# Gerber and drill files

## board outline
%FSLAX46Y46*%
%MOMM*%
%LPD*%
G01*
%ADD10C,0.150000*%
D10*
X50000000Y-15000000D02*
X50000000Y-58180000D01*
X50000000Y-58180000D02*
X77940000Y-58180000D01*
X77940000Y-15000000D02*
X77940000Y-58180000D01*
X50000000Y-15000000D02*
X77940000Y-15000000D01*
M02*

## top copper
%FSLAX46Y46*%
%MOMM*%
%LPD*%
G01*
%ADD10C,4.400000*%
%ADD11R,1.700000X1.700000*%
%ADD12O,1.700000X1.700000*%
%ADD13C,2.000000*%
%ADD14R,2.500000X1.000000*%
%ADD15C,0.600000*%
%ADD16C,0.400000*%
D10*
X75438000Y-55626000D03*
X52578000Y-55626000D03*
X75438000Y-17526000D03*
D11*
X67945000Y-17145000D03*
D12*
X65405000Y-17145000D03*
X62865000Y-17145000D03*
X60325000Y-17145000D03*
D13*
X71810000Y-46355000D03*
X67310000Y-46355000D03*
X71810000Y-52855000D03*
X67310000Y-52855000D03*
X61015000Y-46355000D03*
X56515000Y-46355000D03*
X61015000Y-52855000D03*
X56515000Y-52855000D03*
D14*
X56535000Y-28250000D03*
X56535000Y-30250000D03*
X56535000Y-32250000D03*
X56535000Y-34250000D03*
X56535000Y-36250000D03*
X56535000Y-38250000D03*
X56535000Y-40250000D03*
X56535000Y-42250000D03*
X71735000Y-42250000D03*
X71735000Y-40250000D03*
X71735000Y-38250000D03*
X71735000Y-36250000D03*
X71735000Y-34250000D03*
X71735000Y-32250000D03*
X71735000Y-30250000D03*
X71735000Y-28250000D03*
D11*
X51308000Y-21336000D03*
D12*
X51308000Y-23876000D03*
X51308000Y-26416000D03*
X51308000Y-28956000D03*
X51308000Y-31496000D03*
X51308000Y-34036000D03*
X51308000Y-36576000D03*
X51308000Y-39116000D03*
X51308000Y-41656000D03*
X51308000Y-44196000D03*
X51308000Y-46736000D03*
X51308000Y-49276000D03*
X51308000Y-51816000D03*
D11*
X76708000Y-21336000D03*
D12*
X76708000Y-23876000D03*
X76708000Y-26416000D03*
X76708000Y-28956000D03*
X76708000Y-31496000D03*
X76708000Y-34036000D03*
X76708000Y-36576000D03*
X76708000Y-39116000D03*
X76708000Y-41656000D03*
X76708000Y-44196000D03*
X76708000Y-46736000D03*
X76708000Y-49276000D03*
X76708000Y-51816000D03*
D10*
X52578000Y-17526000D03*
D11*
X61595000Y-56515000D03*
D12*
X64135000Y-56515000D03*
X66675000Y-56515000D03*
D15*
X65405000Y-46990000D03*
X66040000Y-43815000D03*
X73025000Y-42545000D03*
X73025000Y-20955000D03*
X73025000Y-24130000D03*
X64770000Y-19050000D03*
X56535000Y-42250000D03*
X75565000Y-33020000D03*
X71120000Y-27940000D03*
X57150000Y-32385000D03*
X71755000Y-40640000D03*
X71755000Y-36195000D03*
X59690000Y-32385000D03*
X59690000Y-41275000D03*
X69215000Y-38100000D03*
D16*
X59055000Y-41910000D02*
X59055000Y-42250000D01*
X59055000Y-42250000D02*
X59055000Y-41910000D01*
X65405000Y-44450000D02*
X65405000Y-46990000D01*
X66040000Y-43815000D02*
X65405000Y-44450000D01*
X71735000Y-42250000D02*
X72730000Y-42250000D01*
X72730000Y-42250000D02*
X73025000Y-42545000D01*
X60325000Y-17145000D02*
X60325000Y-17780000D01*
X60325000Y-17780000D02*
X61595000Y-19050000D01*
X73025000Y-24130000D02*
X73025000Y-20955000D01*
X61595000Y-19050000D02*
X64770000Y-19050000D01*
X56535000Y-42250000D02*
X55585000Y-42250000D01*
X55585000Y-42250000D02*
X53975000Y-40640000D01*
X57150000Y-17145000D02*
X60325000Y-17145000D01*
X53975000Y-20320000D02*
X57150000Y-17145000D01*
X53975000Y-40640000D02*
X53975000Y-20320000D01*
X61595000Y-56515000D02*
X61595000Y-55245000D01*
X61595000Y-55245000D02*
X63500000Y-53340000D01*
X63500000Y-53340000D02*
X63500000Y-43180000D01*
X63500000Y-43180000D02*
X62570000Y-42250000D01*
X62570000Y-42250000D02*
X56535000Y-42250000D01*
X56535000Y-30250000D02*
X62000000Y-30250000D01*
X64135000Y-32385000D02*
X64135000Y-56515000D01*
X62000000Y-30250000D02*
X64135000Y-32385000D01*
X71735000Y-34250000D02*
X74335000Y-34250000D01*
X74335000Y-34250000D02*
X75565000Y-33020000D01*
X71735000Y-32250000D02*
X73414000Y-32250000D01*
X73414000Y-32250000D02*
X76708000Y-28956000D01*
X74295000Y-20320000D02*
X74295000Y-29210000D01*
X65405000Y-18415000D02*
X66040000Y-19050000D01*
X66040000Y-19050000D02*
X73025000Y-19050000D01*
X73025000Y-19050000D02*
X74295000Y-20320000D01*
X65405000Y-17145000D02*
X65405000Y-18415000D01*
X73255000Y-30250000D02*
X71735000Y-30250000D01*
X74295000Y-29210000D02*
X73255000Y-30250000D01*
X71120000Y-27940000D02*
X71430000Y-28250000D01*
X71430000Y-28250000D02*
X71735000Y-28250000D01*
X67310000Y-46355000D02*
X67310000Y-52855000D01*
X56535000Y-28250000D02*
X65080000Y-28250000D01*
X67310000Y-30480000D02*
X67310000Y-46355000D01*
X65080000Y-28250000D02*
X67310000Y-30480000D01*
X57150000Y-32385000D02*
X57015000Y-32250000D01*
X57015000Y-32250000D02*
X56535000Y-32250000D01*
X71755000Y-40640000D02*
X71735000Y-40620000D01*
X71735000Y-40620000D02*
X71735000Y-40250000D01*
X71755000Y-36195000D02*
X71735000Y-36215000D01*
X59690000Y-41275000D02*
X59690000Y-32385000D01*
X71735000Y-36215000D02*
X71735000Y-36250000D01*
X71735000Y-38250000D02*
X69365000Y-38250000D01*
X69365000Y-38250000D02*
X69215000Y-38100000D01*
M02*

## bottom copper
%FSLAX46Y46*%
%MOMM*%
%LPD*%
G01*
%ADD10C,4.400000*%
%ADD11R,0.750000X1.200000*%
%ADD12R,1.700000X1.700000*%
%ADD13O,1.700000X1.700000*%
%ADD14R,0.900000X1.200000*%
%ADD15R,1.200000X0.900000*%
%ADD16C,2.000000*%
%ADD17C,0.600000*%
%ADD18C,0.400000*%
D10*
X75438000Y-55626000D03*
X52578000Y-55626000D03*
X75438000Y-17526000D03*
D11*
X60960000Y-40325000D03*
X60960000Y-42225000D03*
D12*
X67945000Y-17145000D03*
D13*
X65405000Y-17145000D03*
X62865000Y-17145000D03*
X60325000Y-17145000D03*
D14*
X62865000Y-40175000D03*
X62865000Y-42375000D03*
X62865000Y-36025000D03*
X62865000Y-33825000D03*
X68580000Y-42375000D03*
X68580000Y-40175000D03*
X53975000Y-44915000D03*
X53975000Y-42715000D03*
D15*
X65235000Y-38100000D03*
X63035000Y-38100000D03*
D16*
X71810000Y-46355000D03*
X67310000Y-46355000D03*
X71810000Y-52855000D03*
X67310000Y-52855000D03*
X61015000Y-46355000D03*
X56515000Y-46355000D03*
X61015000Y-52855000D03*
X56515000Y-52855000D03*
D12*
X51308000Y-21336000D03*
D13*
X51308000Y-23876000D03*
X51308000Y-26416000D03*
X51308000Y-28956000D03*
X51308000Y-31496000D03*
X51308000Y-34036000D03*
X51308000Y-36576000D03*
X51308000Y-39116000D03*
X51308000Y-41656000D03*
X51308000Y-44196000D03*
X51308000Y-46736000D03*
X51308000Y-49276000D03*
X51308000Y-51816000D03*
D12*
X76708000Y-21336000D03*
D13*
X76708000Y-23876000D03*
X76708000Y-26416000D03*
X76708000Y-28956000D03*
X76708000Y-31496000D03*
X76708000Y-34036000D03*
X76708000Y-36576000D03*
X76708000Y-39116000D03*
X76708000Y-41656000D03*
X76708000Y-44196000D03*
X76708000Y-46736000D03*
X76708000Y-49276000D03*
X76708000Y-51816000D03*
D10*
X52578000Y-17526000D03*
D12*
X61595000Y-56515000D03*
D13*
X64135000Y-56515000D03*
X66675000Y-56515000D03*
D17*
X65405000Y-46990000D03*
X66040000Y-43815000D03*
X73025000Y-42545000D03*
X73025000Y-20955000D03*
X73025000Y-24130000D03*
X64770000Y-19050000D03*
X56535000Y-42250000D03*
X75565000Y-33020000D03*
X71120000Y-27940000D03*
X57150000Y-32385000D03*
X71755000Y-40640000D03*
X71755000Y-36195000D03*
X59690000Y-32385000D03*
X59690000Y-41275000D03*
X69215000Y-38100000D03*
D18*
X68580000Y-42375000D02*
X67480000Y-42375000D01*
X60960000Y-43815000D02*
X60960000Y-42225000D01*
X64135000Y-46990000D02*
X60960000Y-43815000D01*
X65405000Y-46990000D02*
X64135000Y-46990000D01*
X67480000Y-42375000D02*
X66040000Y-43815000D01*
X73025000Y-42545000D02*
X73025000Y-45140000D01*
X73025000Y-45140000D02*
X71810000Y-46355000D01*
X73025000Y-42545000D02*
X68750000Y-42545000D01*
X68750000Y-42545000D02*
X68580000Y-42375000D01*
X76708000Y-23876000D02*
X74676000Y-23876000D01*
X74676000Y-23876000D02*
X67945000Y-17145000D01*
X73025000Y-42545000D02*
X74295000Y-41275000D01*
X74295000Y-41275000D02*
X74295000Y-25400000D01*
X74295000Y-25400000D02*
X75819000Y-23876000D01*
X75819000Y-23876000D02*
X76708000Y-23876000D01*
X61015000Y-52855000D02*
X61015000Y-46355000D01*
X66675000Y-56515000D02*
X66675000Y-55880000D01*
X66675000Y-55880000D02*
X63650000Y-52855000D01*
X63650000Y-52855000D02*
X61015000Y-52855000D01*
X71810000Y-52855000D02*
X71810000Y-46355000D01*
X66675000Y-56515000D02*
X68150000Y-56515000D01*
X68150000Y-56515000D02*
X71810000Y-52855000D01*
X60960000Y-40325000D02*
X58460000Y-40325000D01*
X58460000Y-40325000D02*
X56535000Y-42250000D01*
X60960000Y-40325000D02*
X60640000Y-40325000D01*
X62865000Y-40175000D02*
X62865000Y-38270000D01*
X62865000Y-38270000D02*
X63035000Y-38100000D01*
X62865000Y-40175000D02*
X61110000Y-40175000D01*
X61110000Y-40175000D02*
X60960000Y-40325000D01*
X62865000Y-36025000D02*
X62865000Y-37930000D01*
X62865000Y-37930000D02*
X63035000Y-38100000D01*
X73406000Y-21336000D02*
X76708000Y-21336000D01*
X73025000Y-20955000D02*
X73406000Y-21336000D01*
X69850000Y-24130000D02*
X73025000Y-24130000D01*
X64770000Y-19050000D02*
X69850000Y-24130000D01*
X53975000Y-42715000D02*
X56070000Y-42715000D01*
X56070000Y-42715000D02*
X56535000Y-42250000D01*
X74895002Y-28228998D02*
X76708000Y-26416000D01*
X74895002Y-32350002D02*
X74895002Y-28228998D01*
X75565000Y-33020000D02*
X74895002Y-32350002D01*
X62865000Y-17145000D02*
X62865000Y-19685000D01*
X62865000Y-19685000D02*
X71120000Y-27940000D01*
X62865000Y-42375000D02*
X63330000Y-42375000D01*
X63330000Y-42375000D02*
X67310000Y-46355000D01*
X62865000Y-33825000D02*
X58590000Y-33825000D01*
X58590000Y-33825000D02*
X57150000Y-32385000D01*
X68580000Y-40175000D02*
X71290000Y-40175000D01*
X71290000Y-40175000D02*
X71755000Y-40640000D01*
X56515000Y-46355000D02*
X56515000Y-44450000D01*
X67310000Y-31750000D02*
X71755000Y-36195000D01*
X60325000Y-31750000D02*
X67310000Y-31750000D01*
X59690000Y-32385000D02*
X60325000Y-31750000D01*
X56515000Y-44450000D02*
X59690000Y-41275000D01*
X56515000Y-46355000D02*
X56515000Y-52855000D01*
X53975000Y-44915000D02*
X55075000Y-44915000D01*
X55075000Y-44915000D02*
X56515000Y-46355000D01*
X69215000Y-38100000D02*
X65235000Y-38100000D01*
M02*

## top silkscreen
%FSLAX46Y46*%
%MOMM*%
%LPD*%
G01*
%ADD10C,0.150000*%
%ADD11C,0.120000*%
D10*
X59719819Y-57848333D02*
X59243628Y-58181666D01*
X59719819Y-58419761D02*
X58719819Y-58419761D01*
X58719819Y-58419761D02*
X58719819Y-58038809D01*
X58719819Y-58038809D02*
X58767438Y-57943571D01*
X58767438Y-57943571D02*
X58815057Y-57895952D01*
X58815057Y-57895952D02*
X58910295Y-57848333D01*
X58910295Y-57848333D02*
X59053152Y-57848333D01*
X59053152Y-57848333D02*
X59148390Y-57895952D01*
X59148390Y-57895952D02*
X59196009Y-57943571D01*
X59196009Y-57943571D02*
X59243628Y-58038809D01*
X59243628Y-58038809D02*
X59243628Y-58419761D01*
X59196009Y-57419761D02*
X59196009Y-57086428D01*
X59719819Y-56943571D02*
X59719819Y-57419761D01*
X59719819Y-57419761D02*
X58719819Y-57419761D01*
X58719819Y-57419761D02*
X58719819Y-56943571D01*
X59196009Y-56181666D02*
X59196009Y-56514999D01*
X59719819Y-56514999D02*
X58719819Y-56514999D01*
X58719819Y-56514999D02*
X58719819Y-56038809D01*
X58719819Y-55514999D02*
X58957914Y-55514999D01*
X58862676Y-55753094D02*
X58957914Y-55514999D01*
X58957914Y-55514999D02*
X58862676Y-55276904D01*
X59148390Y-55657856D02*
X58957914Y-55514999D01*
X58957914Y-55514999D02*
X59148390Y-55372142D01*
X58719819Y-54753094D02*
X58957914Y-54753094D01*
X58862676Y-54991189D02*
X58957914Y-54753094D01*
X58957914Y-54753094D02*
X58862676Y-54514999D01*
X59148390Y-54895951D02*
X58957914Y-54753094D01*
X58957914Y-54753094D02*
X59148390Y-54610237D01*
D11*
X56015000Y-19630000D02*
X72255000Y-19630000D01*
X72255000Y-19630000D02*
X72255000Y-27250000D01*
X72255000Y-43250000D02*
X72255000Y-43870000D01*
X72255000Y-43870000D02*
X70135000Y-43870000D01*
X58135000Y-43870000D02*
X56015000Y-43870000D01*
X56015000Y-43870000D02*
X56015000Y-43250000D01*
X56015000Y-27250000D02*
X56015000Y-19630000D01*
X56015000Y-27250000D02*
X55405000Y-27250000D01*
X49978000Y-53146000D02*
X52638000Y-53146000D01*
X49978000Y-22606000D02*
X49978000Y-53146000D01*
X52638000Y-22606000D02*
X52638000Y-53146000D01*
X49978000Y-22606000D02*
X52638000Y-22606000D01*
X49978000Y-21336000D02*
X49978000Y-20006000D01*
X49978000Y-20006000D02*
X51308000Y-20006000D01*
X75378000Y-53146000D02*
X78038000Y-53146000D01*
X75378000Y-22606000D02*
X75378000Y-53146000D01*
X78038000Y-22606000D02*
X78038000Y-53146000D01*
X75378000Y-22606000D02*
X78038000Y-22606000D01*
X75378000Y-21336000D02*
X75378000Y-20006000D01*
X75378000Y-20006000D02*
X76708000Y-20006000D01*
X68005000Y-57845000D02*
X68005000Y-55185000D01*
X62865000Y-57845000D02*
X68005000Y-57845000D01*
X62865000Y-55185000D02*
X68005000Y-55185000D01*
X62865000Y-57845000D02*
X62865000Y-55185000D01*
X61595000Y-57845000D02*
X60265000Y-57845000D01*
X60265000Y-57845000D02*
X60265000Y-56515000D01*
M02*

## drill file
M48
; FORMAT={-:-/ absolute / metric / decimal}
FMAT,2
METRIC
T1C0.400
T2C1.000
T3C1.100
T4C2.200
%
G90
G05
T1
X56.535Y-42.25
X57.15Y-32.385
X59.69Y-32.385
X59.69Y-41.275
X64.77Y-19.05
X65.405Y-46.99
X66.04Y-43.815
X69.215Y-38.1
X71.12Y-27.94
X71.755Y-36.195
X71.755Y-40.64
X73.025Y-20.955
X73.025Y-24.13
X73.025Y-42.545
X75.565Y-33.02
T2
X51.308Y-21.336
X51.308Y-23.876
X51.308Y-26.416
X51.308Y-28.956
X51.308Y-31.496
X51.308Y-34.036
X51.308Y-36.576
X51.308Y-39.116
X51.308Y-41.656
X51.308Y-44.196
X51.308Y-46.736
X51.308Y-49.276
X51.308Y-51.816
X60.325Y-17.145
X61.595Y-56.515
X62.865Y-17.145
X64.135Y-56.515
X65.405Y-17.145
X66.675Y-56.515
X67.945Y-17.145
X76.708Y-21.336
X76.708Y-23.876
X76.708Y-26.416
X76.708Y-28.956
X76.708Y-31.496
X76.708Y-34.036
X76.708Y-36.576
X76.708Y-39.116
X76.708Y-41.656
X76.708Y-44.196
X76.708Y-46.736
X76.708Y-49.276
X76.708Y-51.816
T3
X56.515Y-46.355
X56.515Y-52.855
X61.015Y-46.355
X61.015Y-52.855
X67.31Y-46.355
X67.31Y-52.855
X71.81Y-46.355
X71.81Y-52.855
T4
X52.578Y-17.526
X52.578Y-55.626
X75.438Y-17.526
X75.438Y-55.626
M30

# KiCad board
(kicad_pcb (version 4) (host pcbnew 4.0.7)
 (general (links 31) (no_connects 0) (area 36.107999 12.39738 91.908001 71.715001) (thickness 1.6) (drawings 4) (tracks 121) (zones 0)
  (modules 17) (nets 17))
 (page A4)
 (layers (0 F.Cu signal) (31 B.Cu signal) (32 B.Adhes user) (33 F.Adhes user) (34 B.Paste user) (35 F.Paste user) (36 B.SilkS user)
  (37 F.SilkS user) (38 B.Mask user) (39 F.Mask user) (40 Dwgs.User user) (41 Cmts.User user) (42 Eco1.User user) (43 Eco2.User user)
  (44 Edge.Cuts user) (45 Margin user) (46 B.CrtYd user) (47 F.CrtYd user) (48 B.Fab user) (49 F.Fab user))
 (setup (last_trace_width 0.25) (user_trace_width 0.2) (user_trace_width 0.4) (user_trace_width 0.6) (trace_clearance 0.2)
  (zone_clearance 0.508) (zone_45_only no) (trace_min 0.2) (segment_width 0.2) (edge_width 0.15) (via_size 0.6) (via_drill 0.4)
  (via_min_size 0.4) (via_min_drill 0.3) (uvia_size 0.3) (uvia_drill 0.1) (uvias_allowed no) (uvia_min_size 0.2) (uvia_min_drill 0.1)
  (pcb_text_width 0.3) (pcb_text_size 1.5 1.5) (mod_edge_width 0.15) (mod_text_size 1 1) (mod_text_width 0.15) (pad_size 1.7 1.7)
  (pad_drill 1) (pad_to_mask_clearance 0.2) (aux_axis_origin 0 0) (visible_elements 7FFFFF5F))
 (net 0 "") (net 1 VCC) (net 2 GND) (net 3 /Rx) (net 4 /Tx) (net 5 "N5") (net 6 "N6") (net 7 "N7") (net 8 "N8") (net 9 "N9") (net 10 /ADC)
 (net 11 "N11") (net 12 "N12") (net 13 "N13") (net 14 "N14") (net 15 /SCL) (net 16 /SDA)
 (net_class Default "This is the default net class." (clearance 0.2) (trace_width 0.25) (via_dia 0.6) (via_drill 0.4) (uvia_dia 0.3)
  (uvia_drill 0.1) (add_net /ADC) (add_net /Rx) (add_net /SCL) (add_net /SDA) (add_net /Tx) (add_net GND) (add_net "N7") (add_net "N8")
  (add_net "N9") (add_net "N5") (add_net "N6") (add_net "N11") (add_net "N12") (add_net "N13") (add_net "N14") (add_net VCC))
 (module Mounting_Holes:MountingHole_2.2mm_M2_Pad (layer F.Cu) (at 75.438 55.626)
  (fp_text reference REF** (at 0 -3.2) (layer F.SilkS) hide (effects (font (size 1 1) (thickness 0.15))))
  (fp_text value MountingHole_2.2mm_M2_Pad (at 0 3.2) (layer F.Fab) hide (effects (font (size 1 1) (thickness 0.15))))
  (pad 1 thru_hole circle (at 0 0) (size 4.4 4.4) (drill 2.2) (layers *.Cu *.Mask)))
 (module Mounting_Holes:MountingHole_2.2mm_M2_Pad (layer F.Cu) (at 52.578 55.626)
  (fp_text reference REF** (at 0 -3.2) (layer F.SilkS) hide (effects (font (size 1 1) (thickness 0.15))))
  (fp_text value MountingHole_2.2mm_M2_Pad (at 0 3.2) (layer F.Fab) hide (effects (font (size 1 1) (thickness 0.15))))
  (pad 1 thru_hole circle (at 0 0) (size 4.4 4.4) (drill 2.2) (layers *.Cu *.Mask)))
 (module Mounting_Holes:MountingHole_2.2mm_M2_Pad (layer F.Cu) (at 75.438 17.526)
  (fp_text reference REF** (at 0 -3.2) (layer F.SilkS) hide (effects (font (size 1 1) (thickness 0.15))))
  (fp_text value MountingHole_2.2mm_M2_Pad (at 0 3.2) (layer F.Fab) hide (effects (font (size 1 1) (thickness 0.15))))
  (pad 1 thru_hole circle (at 0 0) (size 4.4 4.4) (drill 2.2) (layers *.Cu *.Mask)))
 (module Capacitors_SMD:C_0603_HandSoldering (layer B.Cu) (at 60.96 41.275 270)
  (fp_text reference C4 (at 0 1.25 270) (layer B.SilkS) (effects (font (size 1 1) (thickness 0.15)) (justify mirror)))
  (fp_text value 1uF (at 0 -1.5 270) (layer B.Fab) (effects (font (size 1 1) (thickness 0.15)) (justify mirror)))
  (pad 1 smd rect (at -0.95 0 270) (size 1.2 0.75) (layers B.Cu B.Paste B.Mask) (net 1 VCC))
  (pad 2 smd rect (at 0.95 0 270) (size 1.2 0.75) (layers B.Cu B.Paste B.Mask) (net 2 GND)))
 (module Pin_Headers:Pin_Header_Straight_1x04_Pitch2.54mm (layer B.Cu) (at 67.945 17.145 90)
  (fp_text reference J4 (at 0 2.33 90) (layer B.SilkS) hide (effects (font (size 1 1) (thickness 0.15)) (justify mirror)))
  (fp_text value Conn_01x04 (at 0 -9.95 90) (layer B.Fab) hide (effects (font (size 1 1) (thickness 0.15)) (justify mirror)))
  (pad 1 thru_hole rect (at 0 0 90) (size 1.7 1.7) (drill 1) (layers *.Cu *.Mask) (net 2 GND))
  (pad 2 thru_hole oval (at 0 -2.54 90) (size 1.7 1.7) (drill 1) (layers *.Cu *.Mask) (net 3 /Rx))
  (pad 3 thru_hole oval (at 0 -5.08 90) (size 1.7 1.7) (drill 1) (layers *.Cu *.Mask) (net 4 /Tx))
  (pad 4 thru_hole oval (at 0 -7.62 90) (size 1.7 1.7) (drill 1) (layers *.Cu *.Mask) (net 1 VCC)))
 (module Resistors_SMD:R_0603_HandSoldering (layer B.Cu) (at 62.865 41.275 270)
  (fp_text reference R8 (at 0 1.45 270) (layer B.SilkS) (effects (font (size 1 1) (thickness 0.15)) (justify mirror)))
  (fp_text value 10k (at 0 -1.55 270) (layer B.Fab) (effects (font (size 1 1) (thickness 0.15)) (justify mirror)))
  (pad 1 smd rect (at -1.1 0 270) (size 1.2 0.9) (layers B.Cu B.Paste B.Mask) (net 1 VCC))
  (pad 2 smd rect (at 1.1 0 270) (size 1.2 0.9) (layers B.Cu B.Paste B.Mask) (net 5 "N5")))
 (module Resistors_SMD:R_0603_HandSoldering (layer B.Cu) (at 62.865 34.925 90)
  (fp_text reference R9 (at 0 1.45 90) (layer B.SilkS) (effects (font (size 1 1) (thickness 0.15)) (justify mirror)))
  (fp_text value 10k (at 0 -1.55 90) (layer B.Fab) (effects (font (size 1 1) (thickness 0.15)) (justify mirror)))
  (pad 1 smd rect (at -1.1 0 90) (size 1.2 0.9) (layers B.Cu B.Paste B.Mask) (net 1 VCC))
  (pad 2 smd rect (at 1.1 0 90) (size 1.2 0.9) (layers B.Cu B.Paste B.Mask) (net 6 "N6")))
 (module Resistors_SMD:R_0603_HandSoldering (layer B.Cu) (at 68.58 41.275 90)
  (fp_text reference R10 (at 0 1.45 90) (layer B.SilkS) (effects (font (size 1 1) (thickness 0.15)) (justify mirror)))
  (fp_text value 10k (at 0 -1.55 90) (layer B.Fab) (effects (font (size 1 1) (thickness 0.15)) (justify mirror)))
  (pad 1 smd rect (at -1.1 0 90) (size 1.2 0.9) (layers B.Cu B.Paste B.Mask) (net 2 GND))
  (pad 2 smd rect (at 1.1 0 90) (size 1.2 0.9) (layers B.Cu B.Paste B.Mask) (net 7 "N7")))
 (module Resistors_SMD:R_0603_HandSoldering (layer B.Cu) (at 53.975 43.815 90)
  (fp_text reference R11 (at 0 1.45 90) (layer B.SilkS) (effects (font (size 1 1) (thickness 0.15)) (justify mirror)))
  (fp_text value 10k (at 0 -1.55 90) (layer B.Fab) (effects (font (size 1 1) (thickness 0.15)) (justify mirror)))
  (pad 1 smd rect (at -1.1 0 90) (size 1.2 0.9) (layers B.Cu B.Paste B.Mask) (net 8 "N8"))
  (pad 2 smd rect (at 1.1 0 90) (size 1.2 0.9) (layers B.Cu B.Paste B.Mask) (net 1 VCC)))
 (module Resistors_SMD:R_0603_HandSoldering (layer B.Cu) (at 64.135 38.1 180)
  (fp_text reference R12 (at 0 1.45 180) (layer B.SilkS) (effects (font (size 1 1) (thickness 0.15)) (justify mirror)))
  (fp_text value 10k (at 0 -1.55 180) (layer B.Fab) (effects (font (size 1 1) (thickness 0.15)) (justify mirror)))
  (pad 1 smd rect (at -1.1 0 180) (size 1.2 0.9) (layers B.Cu B.Paste B.Mask) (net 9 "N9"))
  (pad 2 smd rect (at 1.1 0 180) (size 1.2 0.9) (layers B.Cu B.Paste B.Mask) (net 1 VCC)))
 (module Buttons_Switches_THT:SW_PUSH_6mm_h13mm (layer B.Cu) (at 67.31 46.355 270)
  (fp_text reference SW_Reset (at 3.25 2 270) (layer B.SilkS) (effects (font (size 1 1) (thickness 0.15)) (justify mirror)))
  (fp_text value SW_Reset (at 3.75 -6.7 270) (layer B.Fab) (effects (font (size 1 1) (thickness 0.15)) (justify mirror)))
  (pad 2 thru_hole circle (at 0 -4.5 180) (size 2 2) (drill 1.1) (layers *.Cu *.Mask) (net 2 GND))
  (pad 1 thru_hole circle (at 0 0 180) (size 2 2) (drill 1.1) (layers *.Cu *.Mask) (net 5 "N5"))
  (pad 2 thru_hole circle (at 6.5 -4.5 180) (size 2 2) (drill 1.1) (layers *.Cu *.Mask) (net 2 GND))
  (pad 1 thru_hole circle (at 6.5 0 180) (size 2 2) (drill 1.1) (layers *.Cu *.Mask) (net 5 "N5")))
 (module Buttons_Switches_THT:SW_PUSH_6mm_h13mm (layer B.Cu) (at 56.515 46.355 270)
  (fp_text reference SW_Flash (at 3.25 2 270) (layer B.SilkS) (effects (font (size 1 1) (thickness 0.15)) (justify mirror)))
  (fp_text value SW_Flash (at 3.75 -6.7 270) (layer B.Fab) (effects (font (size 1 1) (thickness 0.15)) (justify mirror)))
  (pad 2 thru_hole circle (at 0 -4.5 180) (size 2 2) (drill 1.1) (layers *.Cu *.Mask) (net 2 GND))
  (pad 1 thru_hole circle (at 0 0 180) (size 2 2) (drill 1.1) (layers *.Cu *.Mask) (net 8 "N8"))
  (pad 2 thru_hole circle (at 6.5 -4.5 180) (size 2 2) (drill 1.1) (layers *.Cu *.Mask) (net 2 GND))
  (pad 1 thru_hole circle (at 6.5 0 180) (size 2 2) (drill 1.1) (layers *.Cu *.Mask) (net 8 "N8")))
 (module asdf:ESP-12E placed (layer F.Cu) (at 64.135 31.75)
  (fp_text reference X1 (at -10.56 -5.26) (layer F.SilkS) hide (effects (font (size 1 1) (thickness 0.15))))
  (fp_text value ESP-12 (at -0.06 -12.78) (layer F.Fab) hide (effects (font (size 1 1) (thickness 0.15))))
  (fp_line (start -8.12 -12.12) (end 8.12 -12.12) (layer F.SilkS) (width 0.12))
  (fp_line (start 8.12 -12.12) (end 8.12 -4.5) (layer F.SilkS) (width 0.12))
  (fp_line (start 8.12 11.5) (end 8.12 12.12) (layer F.SilkS) (width 0.12))
  (fp_line (start 8.12 12.12) (end 6 12.12) (layer F.SilkS) (width 0.12))
  (fp_line (start -6 12.12) (end -8.12 12.12) (layer F.SilkS) (width 0.12))
  (fp_line (start -8.12 12.12) (end -8.12 11.5) (layer F.SilkS) (width 0.12))
  (fp_line (start -8.12 -4.5) (end -8.12 -12.12) (layer F.SilkS) (width 0.12))
  (fp_line (start -8.12 -4.5) (end -8.73 -4.5) (layer F.SilkS) (width 0.12))
  (pad 1 smd rect (at -7.6 -3.5) (size 2.5 1) (layers F.Cu F.Paste F.Mask) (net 5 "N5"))
  (pad 2 smd rect (at -7.6 -1.5) (size 2.5 1) (layers F.Cu F.Paste F.Mask) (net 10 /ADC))
  (pad 3 smd rect (at -7.6 0.5) (size 2.5 1) (layers F.Cu F.Paste F.Mask) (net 6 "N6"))
  (pad 4 smd rect (at -7.6 2.5) (size 2.5 1) (layers F.Cu F.Paste F.Mask) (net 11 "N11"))
  (pad 5 smd rect (at -7.6 4.5) (size 2.5 1) (layers F.Cu F.Paste F.Mask) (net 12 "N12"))
  (pad 6 smd rect (at -7.6 6.5) (size 2.5 1) (layers F.Cu F.Paste F.Mask) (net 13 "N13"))
  (pad 7 smd rect (at -7.6 8.5) (size 2.5 1) (layers F.Cu F.Paste F.Mask) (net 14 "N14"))
  (pad 8 smd rect (at -7.6 10.5) (size 2.5 1) (layers F.Cu F.Paste F.Mask) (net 1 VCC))
  (pad 9 smd rect (at 7.6 10.5) (size 2.5 1) (layers F.Cu F.Paste F.Mask) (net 2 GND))
  (pad 10 smd rect (at 7.6 8.5) (size 2.5 1) (layers F.Cu F.Paste F.Mask) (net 7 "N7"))
  (pad 11 smd rect (at 7.6 6.5) (size 2.5 1) (layers F.Cu F.Paste F.Mask) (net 9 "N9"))
  (pad 12 smd rect (at 7.6 4.5) (size 2.5 1) (layers F.Cu F.Paste F.Mask) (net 8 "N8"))
  (pad 13 smd rect (at 7.6 2.5) (size 2.5 1) (layers F.Cu F.Paste F.Mask) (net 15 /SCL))
  (pad 14 smd rect (at 7.6 0.5) (size 2.5 1) (layers F.Cu F.Paste F.Mask) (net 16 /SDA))
  (pad 15 smd rect (at 7.6 -1.5) (size 2.5 1) (layers F.Cu F.Paste F.Mask) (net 3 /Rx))
  (pad 16 smd rect (at 7.6 -3.5) (size 2.5 1) (layers F.Cu F.Paste F.Mask) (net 4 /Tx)))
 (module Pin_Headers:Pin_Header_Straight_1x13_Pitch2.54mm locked (layer F.Cu) (at 51.308 21.336)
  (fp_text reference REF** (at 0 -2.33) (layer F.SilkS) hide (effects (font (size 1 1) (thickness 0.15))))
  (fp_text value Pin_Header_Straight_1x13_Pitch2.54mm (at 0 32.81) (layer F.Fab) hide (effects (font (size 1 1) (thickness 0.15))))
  (fp_line (start -1.33 31.81) (end 1.33 31.81) (layer F.SilkS) (width 0.12))
  (fp_line (start -1.33 1.27) (end -1.33 31.81) (layer F.SilkS) (width 0.12))
  (fp_line (start 1.33 1.27) (end 1.33 31.81) (layer F.SilkS) (width 0.12))
  (fp_line (start -1.33 1.27) (end 1.33 1.27) (layer F.SilkS) (width 0.12))
  (fp_line (start -1.33 0) (end -1.33 -1.33) (layer F.SilkS) (width 0.12))
  (fp_line (start -1.33 -1.33) (end 0 -1.33) (layer F.SilkS) (width 0.12))
  (pad 1 thru_hole rect (at 0 0) (size 1.7 1.7) (drill 1) (layers *.Cu *.Mask))
  (pad 2 thru_hole oval (at 0 2.54) (size 1.7 1.7) (drill 1) (layers *.Cu *.Mask))
  (pad 3 thru_hole oval (at 0 5.08) (size 1.7 1.7) (drill 1) (layers *.Cu *.Mask))
  (pad 4 thru_hole oval (at 0 7.62) (size 1.7 1.7) (drill 1) (layers *.Cu *.Mask))
  (pad 5 thru_hole oval (at 0 10.16) (size 1.7 1.7) (drill 1) (layers *.Cu *.Mask))
  (pad 6 thru_hole oval (at 0 12.7) (size 1.7 1.7) (drill 1) (layers *.Cu *.Mask))
  (pad 7 thru_hole oval (at 0 15.24) (size 1.7 1.7) (drill 1) (layers *.Cu *.Mask))
  (pad 8 thru_hole oval (at 0 17.78) (size 1.7 1.7) (drill 1) (layers *.Cu *.Mask))
  (pad 9 thru_hole oval (at 0 20.32) (size 1.7 1.7) (drill 1) (layers *.Cu *.Mask))
  (pad 10 thru_hole oval (at 0 22.86) (size 1.7 1.7) (drill 1) (layers *.Cu *.Mask))
  (pad 11 thru_hole oval (at 0 25.4) (size 1.7 1.7) (drill 1) (layers *.Cu *.Mask))
  (pad 12 thru_hole oval (at 0 27.94) (size 1.7 1.7) (drill 1) (layers *.Cu *.Mask))
  (pad 13 thru_hole oval (at 0 30.48) (size 1.7 1.7) (drill 1) (layers *.Cu *.Mask)))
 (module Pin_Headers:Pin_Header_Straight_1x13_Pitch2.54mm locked (layer F.Cu) (at 76.708 21.336)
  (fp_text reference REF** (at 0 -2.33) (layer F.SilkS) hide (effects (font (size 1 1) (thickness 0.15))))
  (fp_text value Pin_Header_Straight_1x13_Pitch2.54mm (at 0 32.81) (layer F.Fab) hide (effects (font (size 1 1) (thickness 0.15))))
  (fp_line (start -1.33 31.81) (end 1.33 31.81) (layer F.SilkS) (width 0.12))
  (fp_line (start -1.33 1.27) (end -1.33 31.81) (layer F.SilkS) (width 0.12))
  (fp_line (start 1.33 1.27) (end 1.33 31.81) (layer F.SilkS) (width 0.12))
  (fp_line (start -1.33 1.27) (end 1.33 1.27) (layer F.SilkS) (width 0.12))
  (fp_line (start -1.33 0) (end -1.33 -1.33) (layer F.SilkS) (width 0.12))
  (fp_line (start -1.33 -1.33) (end 0 -1.33) (layer F.SilkS) (width 0.12))
  (pad 1 thru_hole rect (at 0 0) (size 1.7 1.7) (drill 1) (layers *.Cu *.Mask) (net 1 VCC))
  (pad 2 thru_hole oval (at 0 2.54) (size 1.7 1.7) (drill 1) (layers *.Cu *.Mask) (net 2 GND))
  (pad 3 thru_hole oval (at 0 5.08) (size 1.7 1.7) (drill 1) (layers *.Cu *.Mask) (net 15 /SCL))
  (pad 4 thru_hole oval (at 0 7.62) (size 1.7 1.7) (drill 1) (layers *.Cu *.Mask) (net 16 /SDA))
  (pad 5 thru_hole oval (at 0 10.16) (size 1.7 1.7) (drill 1) (layers *.Cu *.Mask))
  (pad 6 thru_hole oval (at 0 12.7) (size 1.7 1.7) (drill 1) (layers *.Cu *.Mask))
  (pad 7 thru_hole oval (at 0 15.24) (size 1.7 1.7) (drill 1) (layers *.Cu *.Mask))
  (pad 8 thru_hole oval (at 0 17.78) (size 1.7 1.7) (drill 1) (layers *.Cu *.Mask))
  (pad 9 thru_hole oval (at 0 20.32) (size 1.7 1.7) (drill 1) (layers *.Cu *.Mask))
  (pad 10 thru_hole oval (at 0 22.86) (size 1.7 1.7) (drill 1) (layers *.Cu *.Mask))
  (pad 11 thru_hole oval (at 0 25.4) (size 1.7 1.7) (drill 1) (layers *.Cu *.Mask))
  (pad 12 thru_hole oval (at 0 27.94) (size 1.7 1.7) (drill 1) (layers *.Cu *.Mask))
  (pad 13 thru_hole oval (at 0 30.48) (size 1.7 1.7) (drill 1) (layers *.Cu *.Mask)))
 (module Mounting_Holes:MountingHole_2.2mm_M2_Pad (layer F.Cu) (at 52.578 17.526)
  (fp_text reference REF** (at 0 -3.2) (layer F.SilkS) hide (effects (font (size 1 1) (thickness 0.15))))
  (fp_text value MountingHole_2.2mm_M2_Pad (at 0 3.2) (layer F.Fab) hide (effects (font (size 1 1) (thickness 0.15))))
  (pad 1 thru_hole circle (at 0 0) (size 4.4 4.4) (drill 2.2) (layers *.Cu *.Mask)))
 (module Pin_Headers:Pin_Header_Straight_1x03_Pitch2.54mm (layer F.Cu) (at 61.595 56.515 90)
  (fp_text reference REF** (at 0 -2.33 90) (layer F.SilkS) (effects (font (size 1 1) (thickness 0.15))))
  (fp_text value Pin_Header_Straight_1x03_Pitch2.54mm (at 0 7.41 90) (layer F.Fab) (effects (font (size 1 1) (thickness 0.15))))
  (fp_line (start -1.33 6.41) (end 1.33 6.41) (layer F.SilkS) (width 0.12))
  (fp_line (start -1.33 1.27) (end -1.33 6.41) (layer F.SilkS) (width 0.12))
  (fp_line (start 1.33 1.27) (end 1.33 6.41) (layer F.SilkS) (width 0.12))
  (fp_line (start -1.33 1.27) (end 1.33 1.27) (layer F.SilkS) (width 0.12))
  (fp_line (start -1.33 0) (end -1.33 -1.33) (layer F.SilkS) (width 0.12))
  (fp_line (start -1.33 -1.33) (end 0 -1.33) (layer F.SilkS) (width 0.12))
  (pad 1 thru_hole rect (at 0 0 90) (size 1.7 1.7) (drill 1) (layers *.Cu *.Mask) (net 1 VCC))
  (pad 2 thru_hole oval (at 0 2.54 90) (size 1.7 1.7) (drill 1) (layers *.Cu *.Mask) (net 10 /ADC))
  (pad 3 thru_hole oval (at 0 5.08 90) (size 1.7 1.7) (drill 1) (layers *.Cu *.Mask) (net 2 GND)))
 (gr_line (start 50 15) (end 50 58.18) (angle 90) (layer Edge.Cuts) (width 0.15))
 (gr_line (start 50 58.18) (end 77.94 58.18) (angle 90) (layer Edge.Cuts) (width 0.15))
 (gr_line (start 77.94 15) (end 77.94 58.18) (angle 90) (layer Edge.Cuts) (width 0.15))
 (gr_line (start 50 15) (end 77.94 15) (angle 90) (layer Edge.Cuts) (width 0.15))
 (segment (start 59.055 41.91) (end 59.055 42.25) (width 0.4) (layer F.Cu) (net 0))
 (segment (start 59.055 42.25) (end 59.055 41.91) (width 0.4) (layer F.Cu) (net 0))
 (segment (start 68.58 42.375) (end 67.48 42.375) (width 0.4) (layer B.Cu) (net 2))
 (segment (start 60.96 43.815) (end 60.96 42.225) (width 0.4) (layer B.Cu) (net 2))
 (segment (start 64.135 46.99) (end 60.96 43.815) (width 0.4) (layer B.Cu) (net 2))
 (segment (start 65.405 46.99) (end 64.135 46.99) (width 0.4) (layer B.Cu) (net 2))
 (via (at 65.405 46.99) (size 0.6) (drill 0.4) (layers F.Cu B.Cu) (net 2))
 (segment (start 65.405 44.45) (end 65.405 46.99) (width 0.4) (layer F.Cu) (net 2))
 (segment (start 66.04 43.815) (end 65.405 44.45) (width 0.4) (layer F.Cu) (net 2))
 (via (at 66.04 43.815) (size 0.6) (drill 0.4) (layers F.Cu B.Cu) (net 2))
 (segment (start 67.48 42.375) (end 66.04 43.815) (width 0.4) (layer B.Cu) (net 2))
 (segment (start 73.025 42.545) (end 73.025 45.14) (width 0.4) (layer B.Cu) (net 2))
 (segment (start 73.025 45.14) (end 71.81 46.355) (width 0.4) (layer B.Cu) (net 2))
 (segment (start 73.025 42.545) (end 68.75 42.545) (width 0.4) (layer B.Cu) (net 2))
 (segment (start 68.75 42.545) (end 68.58 42.375) (width 0.4) (layer B.Cu) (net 2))
 (segment (start 76.708 23.876) (end 74.676 23.876) (width 0.4) (layer B.Cu) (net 2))
 (segment (start 74.676 23.876) (end 67.945 17.145) (width 0.4) (layer B.Cu) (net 2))
 (segment (start 71.735 42.25) (end 72.73 42.25) (width 0.4) (layer F.Cu) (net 2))
 (segment (start 72.73 42.25) (end 73.025 42.545) (width 0.4) (layer F.Cu) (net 2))
 (via (at 73.025 42.545) (size 0.6) (drill 0.4) (layers F.Cu B.Cu) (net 2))
 (segment (start 73.025 42.545) (end 74.295 41.275) (width 0.4) (layer B.Cu) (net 2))
 (segment (start 74.295 41.275) (end 74.295 25.4) (width 0.4) (layer B.Cu) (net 2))
 (segment (start 74.295 25.4) (end 75.819 23.876) (width 0.4) (layer B.Cu) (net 2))
 (segment (start 75.819 23.876) (end 76.708 23.876) (width 0.4) (layer B.Cu) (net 2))
 (segment (start 61.015 52.855) (end 61.015 46.355) (width 0.4) (layer B.Cu) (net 2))
 (segment (start 66.675 56.515) (end 66.675 55.88) (width 0.4) (layer B.Cu) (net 2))
 (segment (start 66.675 55.88) (end 63.65 52.855) (width 0.4) (layer B.Cu) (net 2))
 (segment (start 63.65 52.855) (end 61.015 52.855) (width 0.4) (layer B.Cu) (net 2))
 (segment (start 71.81 52.855) (end 71.81 46.355) (width 0.4) (layer B.Cu) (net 2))
 (segment (start 66.675 56.515) (end 68.15 56.515) (width 0.4) (layer B.Cu) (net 2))
 (segment (start 68.15 56.515) (end 71.81 52.855) (width 0.4) (layer B.Cu) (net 2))
 (segment (start 60.96 40.325) (end 58.46 40.325) (width 0.4) (layer B.Cu) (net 1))
 (segment (start 58.46 40.325) (end 56.535 42.25) (width 0.4) (layer B.Cu) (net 1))
 (segment (start 60.96 40.325) (end 60.64 40.325) (width 0.4) (layer B.Cu) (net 1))
 (segment (start 62.865 40.175) (end 62.865 38.27) (width 0.4) (layer B.Cu) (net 1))
 (segment (start 62.865 38.27) (end 63.035 38.1) (width 0.4) (layer B.Cu) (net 1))
 (segment (start 62.865 40.175) (end 61.11 40.175) (width 0.4) (layer B.Cu) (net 1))
 (segment (start 61.11 40.175) (end 60.96 40.325) (width 0.4) (layer B.Cu) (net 1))
 (segment (start 62.865 36.025) (end 62.865 37.93) (width 0.4) (layer B.Cu) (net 1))
 (segment (start 62.865 37.93) (end 63.035 38.1) (width 0.4) (layer B.Cu) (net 1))
 (segment (start 60.325 17.145) (end 60.325 17.78) (width 0.4) (layer F.Cu) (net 1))
 (segment (start 60.325 17.78) (end 61.595 19.05) (width 0.4) (layer F.Cu) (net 1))
 (segment (start 73.406 21.336) (end 76.708 21.336) (width 0.4) (layer B.Cu) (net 1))
 (segment (start 73.025 20.955) (end 73.406 21.336) (width 0.4) (layer B.Cu) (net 1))
 (via (at 73.025 20.955) (size 0.6) (drill 0.4) (layers F.Cu B.Cu) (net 1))
 (segment (start 73.025 24.13) (end 73.025 20.955) (width 0.4) (layer F.Cu) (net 1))
 (via (at 73.025 24.13) (size 0.6) (drill 0.4) (layers F.Cu B.Cu) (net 1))
 (segment (start 69.85 24.13) (end 73.025 24.13) (width 0.4) (layer B.Cu) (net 1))
 (segment (start 64.77 19.05) (end 69.85 24.13) (width 0.4) (layer B.Cu) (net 1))
 (via (at 64.77 19.05) (size 0.6) (drill 0.4) (layers F.Cu B.Cu) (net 1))
 (segment (start 61.595 19.05) (end 64.77 19.05) (width 0.4) (layer F.Cu) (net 1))
 (via (at 56.535 42.25) (size 0.6) (drill 0.4) (layers F.Cu B.Cu) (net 1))
 (segment (start 53.975 42.715) (end 56.07 42.715) (width 0.4) (layer B.Cu) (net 1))
 (segment (start 56.07 42.715) (end 56.535 42.25) (width 0.4) (layer B.Cu) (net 1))
 (segment (start 56.535 42.25) (end 55.585 42.25) (width 0.4) (layer F.Cu) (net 1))
 (segment (start 55.585 42.25) (end 53.975 40.64) (width 0.4) (layer F.Cu) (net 1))
 (segment (start 57.15 17.145) (end 60.325 17.145) (width 0.4) (layer F.Cu) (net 1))
 (segment (start 53.975 20.32) (end 57.15 17.145) (width 0.4) (layer F.Cu) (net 1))
 (segment (start 53.975 40.64) (end 53.975 20.32) (width 0.4) (layer F.Cu) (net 1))
 (segment (start 61.595 56.515) (end 61.595 55.245) (width 0.4) (layer F.Cu) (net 1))
 (segment (start 61.595 55.245) (end 63.5 53.34) (width 0.4) (layer F.Cu) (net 1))
 (segment (start 63.5 53.34) (end 63.5 43.18) (width 0.4) (layer F.Cu) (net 1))
 (segment (start 63.5 43.18) (end 62.57 42.25) (width 0.4) (layer F.Cu) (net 1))
 (segment (start 62.57 42.25) (end 56.535 42.25) (width 0.4) (layer F.Cu) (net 1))
 (segment (start 56.535 30.25) (end 62 30.25) (width 0.4) (layer F.Cu) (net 10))
 (segment (start 64.135 32.385) (end 64.135 56.515) (width 0.4) (layer F.Cu) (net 10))
 (segment (start 62 30.25) (end 64.135 32.385) (width 0.4) (layer F.Cu) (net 10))
 (segment (start 71.735 34.25) (end 74.335 34.25) (width 0.4) (layer F.Cu) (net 15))
 (segment (start 74.895002 28.228998) (end 76.708 26.416) (width 0.4) (layer B.Cu) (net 15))
 (segment (start 74.895002 32.350002) (end 74.895002 28.228998) (width 0.4) (layer B.Cu) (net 15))
 (segment (start 75.565 33.02) (end 74.895002 32.350002) (width 0.4) (layer B.Cu) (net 15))
 (via (at 75.565 33.02) (size 0.6) (drill 0.4) (layers F.Cu B.Cu) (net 15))
 (segment (start 74.335 34.25) (end 75.565 33.02) (width 0.4) (layer F.Cu) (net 15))
 (segment (start 71.735 32.25) (end 73.414 32.25) (width 0.4) (layer F.Cu) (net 16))
 (segment (start 73.414 32.25) (end 76.708 28.956) (width 0.4) (layer F.Cu) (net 16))
 (segment (start 74.295 20.32) (end 74.295 29.21) (width 0.4) (layer F.Cu) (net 3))
 (segment (start 65.405 18.415) (end 66.04 19.05) (width 0.4) (layer F.Cu) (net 3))
 (segment (start 66.04 19.05) (end 73.025 19.05) (width 0.4) (layer F.Cu) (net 3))
 (segment (start 73.025 19.05) (end 74.295 20.32) (width 0.4) (layer F.Cu) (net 3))
 (segment (start 65.405 17.145) (end 65.405 18.415) (width 0.4) (layer F.Cu) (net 3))
 (segment (start 73.255 30.25) (end 71.735 30.25) (width 0.4) (layer F.Cu) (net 3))
 (segment (start 74.295 29.21) (end 73.255 30.25) (width 0.4) (layer F.Cu) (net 3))
 (segment (start 62.865 17.145) (end 62.865 19.685) (width 0.4) (layer B.Cu) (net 4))
 (segment (start 71.12 27.94) (end 71.43 28.25) (width 0.4) (layer F.Cu) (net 4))
 (via (at 71.12 27.94) (size 0.6) (drill 0.4) (layers F.Cu B.Cu) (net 4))
 (segment (start 62.865 19.685) (end 71.12 27.94) (width 0.4) (layer B.Cu) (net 4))
 (segment (start 71.43 28.25) (end 71.735 28.25) (width 0.4) (layer F.Cu) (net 4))
 (segment (start 62.865 42.375) (end 63.33 42.375) (width 0.4) (layer B.Cu) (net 5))
 (segment (start 63.33 42.375) (end 67.31 46.355) (width 0.4) (layer B.Cu) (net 5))
 (segment (start 67.31 46.355) (end 67.31 52.855) (width 0.4) (layer F.Cu) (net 5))
 (segment (start 56.535 28.25) (end 65.08 28.25) (width 0.4) (layer F.Cu) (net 5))
 (segment (start 67.31 30.48) (end 67.31 46.355) (width 0.4) (layer F.Cu) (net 5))
 (segment (start 65.08 28.25) (end 67.31 30.48) (width 0.4) (layer F.Cu) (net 5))
 (segment (start 62.865 33.825) (end 58.59 33.825) (width 0.4) (layer B.Cu) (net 6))
 (segment (start 57.15 32.385) (end 57.015 32.25) (width 0.4) (layer F.Cu) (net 6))
 (via (at 57.15 32.385) (size 0.6) (drill 0.4) (layers F.Cu B.Cu) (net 6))
 (segment (start 58.59 33.825) (end 57.15 32.385) (width 0.4) (layer B.Cu) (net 6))
 (segment (start 57.015 32.25) (end 56.535 32.25) (width 0.4) (layer F.Cu) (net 6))
 (segment (start 68.58 40.175) (end 71.29 40.175) (width 0.4) (layer B.Cu) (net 7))
 (segment (start 71.755 40.64) (end 71.735 40.62) (width 0.4) (layer F.Cu) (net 7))
 (via (at 71.755 40.64) (size 0.6) (drill 0.4) (layers F.Cu B.Cu) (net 7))
 (segment (start 71.29 40.175) (end 71.755 40.64) (width 0.4) (layer B.Cu) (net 7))
 (segment (start 71.735 40.62) (end 71.735 40.25) (width 0.4) (layer F.Cu) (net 7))
 (segment (start 56.515 46.355) (end 56.515 44.45) (width 0.4) (layer B.Cu) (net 8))
 (segment (start 71.755 36.195) (end 71.735 36.215) (width 0.4) (layer F.Cu) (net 8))
 (via (at 71.755 36.195) (size 0.6) (drill 0.4) (layers F.Cu B.Cu) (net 8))
 (segment (start 67.31 31.75) (end 71.755 36.195) (width 0.4) (layer B.Cu) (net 8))
 (segment (start 60.325 31.75) (end 67.31 31.75) (width 0.4) (layer B.Cu) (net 8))
 (segment (start 59.69 32.385) (end 60.325 31.75) (width 0.4) (layer B.Cu) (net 8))
 (via (at 59.69 32.385) (size 0.6) (drill 0.4) (layers F.Cu B.Cu) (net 8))
 (segment (start 59.69 41.275) (end 59.69 32.385) (width 0.4) (layer F.Cu) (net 8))
 (via (at 59.69 41.275) (size 0.6) (drill 0.4) (layers F.Cu B.Cu) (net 8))
 (segment (start 56.515 44.45) (end 59.69 41.275) (width 0.4) (layer B.Cu) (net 8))
 (segment (start 71.735 36.215) (end 71.735 36.25) (width 0.4) (layer F.Cu) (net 8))
 (segment (start 56.515 46.355) (end 56.515 52.855) (width 0.4) (layer B.Cu) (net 8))
 (segment (start 53.975 44.915) (end 55.075 44.915) (width 0.4) (layer B.Cu) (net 8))
 (segment (start 55.075 44.915) (end 56.515 46.355) (width 0.4) (layer B.Cu) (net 8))
 (segment (start 71.735 38.25) (end 69.365 38.25) (width 0.4) (layer F.Cu) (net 9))
 (segment (start 69.215 38.1) (end 65.235 38.1) (width 0.4) (layer B.Cu) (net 9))
 (via (at 69.215 38.1) (size 0.6) (drill 0.4) (layers F.Cu B.Cu) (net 9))
 (segment (start 69.365 38.25) (end 69.215 38.1) (width 0.4) (layer F.Cu) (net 9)))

